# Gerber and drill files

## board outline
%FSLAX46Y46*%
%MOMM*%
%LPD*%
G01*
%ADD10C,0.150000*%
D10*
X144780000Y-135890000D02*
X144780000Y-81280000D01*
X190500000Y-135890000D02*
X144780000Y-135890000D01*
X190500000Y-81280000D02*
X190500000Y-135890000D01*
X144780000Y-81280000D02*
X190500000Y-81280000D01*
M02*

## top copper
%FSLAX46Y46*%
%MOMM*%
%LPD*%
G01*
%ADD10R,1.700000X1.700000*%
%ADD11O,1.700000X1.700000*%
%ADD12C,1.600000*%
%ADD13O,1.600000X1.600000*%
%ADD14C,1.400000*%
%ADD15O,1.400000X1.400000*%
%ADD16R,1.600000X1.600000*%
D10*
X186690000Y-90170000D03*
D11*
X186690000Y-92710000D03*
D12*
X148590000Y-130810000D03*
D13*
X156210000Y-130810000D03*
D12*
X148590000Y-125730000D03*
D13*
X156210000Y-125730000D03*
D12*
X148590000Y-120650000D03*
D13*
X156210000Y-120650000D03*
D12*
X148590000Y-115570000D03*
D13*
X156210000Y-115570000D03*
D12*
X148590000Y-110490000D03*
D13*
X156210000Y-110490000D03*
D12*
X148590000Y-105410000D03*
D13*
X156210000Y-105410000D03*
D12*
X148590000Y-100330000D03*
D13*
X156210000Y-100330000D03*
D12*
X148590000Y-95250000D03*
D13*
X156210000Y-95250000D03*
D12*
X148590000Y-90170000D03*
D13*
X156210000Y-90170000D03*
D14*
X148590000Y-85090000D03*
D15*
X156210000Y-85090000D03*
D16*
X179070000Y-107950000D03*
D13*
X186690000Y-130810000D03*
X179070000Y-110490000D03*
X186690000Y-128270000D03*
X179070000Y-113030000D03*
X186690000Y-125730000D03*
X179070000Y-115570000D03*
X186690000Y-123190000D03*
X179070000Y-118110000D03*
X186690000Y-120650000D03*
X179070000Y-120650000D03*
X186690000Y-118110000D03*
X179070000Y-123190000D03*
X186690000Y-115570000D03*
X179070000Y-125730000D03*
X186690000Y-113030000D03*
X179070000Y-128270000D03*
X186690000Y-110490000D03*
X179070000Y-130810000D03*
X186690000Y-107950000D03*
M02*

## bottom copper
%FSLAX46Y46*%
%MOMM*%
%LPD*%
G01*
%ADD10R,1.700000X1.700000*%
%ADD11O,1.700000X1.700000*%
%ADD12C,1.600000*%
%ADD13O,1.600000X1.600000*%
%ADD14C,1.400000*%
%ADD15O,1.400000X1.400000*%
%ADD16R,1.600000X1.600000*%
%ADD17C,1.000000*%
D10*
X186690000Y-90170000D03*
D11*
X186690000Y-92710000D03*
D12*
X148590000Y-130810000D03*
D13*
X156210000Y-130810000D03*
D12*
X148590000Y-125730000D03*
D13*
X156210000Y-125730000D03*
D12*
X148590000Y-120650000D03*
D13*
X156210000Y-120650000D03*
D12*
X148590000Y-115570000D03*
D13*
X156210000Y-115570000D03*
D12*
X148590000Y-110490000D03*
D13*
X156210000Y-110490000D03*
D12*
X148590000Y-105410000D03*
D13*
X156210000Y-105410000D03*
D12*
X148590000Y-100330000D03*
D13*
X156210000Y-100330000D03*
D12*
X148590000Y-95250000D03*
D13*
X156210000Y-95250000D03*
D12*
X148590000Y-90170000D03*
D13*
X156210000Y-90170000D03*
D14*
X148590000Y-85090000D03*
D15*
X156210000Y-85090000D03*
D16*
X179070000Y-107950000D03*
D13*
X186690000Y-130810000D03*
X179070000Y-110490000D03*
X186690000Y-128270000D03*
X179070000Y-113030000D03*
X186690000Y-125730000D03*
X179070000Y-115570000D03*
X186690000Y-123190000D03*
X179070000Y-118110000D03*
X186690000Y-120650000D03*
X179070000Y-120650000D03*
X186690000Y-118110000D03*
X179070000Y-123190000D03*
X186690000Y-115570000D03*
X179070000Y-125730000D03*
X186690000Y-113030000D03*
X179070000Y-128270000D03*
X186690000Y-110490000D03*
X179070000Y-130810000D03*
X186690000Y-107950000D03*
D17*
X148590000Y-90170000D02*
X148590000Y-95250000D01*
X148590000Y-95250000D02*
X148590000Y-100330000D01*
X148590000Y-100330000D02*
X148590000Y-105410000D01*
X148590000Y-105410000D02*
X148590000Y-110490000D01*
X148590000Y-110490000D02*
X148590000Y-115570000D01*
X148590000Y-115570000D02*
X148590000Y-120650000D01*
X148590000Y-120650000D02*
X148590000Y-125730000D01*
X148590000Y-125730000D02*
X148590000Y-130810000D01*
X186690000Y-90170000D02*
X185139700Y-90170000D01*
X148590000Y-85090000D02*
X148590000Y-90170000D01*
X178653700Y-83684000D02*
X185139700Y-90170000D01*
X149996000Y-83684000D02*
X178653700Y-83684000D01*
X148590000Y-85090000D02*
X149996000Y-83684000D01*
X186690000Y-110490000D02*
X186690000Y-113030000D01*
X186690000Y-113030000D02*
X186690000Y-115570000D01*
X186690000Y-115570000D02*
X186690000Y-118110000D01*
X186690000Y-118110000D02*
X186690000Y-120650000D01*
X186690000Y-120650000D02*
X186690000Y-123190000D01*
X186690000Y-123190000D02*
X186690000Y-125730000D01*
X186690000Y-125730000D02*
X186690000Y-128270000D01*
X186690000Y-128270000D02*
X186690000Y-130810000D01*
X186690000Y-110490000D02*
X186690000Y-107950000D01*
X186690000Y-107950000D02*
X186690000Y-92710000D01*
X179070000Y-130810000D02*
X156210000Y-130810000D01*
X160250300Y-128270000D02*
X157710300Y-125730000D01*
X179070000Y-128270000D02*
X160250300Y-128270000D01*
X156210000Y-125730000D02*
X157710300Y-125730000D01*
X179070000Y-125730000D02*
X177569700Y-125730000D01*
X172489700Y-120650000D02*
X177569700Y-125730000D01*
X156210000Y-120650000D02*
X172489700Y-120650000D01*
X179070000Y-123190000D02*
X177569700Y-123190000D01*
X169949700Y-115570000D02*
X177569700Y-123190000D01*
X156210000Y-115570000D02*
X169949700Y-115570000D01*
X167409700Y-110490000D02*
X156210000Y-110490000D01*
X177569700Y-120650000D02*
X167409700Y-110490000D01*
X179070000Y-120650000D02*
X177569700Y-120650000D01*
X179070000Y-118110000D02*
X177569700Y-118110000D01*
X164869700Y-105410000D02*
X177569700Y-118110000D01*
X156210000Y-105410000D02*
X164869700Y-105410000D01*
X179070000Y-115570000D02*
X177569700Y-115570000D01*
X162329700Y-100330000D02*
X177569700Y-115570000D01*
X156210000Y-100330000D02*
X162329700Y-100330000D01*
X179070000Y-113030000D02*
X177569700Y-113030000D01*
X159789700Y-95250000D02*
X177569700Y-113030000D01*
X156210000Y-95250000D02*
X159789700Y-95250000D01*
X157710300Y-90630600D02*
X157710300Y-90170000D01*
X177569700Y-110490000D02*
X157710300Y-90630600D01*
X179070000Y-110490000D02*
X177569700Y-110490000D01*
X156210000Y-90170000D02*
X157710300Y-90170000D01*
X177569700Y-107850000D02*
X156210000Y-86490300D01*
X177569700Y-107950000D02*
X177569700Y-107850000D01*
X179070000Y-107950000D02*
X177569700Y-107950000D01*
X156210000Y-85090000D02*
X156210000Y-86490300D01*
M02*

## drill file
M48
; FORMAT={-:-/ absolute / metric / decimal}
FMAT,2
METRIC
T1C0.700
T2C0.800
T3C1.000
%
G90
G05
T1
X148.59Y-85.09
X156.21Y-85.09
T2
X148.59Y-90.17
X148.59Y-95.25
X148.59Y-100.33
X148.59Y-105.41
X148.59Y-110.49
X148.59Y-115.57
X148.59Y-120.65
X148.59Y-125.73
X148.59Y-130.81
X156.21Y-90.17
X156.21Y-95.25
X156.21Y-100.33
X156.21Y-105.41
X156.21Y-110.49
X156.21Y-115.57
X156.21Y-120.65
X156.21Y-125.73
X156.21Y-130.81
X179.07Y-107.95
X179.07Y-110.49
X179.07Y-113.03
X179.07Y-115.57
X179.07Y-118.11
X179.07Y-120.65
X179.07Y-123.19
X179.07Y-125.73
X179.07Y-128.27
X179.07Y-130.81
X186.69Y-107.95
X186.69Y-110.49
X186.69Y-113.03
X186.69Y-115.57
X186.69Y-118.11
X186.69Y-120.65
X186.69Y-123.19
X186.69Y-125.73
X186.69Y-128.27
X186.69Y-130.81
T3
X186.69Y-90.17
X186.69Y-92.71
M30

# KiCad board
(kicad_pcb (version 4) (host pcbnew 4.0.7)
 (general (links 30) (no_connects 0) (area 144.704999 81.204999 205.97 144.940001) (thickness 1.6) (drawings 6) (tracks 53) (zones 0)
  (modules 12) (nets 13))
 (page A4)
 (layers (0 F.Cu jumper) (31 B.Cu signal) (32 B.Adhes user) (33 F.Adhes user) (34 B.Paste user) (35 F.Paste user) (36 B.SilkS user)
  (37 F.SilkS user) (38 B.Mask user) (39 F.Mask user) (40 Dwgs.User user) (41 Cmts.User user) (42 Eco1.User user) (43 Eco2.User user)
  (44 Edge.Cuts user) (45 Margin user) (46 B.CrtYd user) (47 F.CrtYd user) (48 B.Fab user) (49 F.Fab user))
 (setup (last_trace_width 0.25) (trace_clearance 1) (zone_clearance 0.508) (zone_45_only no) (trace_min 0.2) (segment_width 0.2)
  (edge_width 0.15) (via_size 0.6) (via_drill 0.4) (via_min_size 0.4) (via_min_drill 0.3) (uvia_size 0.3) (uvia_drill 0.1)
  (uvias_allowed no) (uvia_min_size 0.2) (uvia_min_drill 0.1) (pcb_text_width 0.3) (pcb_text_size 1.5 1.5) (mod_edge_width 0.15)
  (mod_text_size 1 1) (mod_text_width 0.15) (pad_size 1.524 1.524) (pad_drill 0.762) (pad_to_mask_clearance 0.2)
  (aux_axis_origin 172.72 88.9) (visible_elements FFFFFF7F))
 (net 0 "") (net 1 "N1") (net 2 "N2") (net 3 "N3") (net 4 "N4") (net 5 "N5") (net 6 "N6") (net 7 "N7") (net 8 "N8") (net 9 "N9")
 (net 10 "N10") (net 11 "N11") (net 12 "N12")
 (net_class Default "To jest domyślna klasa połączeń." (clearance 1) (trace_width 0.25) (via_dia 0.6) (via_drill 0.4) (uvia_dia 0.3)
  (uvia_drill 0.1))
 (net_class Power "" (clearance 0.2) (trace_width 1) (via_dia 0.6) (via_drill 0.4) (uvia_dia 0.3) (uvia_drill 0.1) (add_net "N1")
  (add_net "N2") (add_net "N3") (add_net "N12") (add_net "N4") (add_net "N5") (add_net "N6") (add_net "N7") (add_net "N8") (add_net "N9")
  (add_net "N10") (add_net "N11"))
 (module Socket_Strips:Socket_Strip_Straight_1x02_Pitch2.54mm (layer F.Cu) (at 186.69 90.17)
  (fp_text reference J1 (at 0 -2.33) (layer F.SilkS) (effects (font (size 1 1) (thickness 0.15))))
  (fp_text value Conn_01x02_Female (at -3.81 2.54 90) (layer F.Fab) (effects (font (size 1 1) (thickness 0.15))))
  (pad 1 thru_hole rect (at 0 0) (size 1.7 1.7) (drill 1) (layers *.Cu *.Mask) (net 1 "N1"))
  (pad 2 thru_hole oval (at 0 2.54) (size 1.7 1.7) (drill 1) (layers *.Cu *.Mask) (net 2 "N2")))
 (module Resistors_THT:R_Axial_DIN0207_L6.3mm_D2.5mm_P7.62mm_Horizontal (layer F.Cu) (at 148.59 130.81)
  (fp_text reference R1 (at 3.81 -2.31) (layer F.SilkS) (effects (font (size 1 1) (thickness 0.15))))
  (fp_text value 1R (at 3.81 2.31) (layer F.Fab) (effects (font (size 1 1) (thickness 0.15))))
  (pad 1 thru_hole circle (at 0 0) (size 1.6 1.6) (drill 0.8) (layers *.Cu *.Mask) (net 1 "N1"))
  (pad 2 thru_hole oval (at 7.62 0) (size 1.6 1.6) (drill 0.8) (layers *.Cu *.Mask) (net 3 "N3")))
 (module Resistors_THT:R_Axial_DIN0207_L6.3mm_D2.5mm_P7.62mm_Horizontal (layer F.Cu) (at 148.59 125.73)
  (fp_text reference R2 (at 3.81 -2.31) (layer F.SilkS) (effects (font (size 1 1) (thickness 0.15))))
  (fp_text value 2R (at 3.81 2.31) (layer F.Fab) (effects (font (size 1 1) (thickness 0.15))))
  (pad 1 thru_hole circle (at 0 0) (size 1.6 1.6) (drill 0.8) (layers *.Cu *.Mask) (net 1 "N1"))
  (pad 2 thru_hole oval (at 7.62 0) (size 1.6 1.6) (drill 0.8) (layers *.Cu *.Mask) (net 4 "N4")))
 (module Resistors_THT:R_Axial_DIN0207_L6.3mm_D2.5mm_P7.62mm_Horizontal (layer F.Cu) (at 148.59 120.65)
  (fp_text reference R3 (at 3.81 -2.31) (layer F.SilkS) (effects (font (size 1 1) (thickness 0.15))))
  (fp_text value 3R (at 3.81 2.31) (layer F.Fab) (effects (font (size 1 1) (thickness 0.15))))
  (pad 1 thru_hole circle (at 0 0) (size 1.6 1.6) (drill 0.8) (layers *.Cu *.Mask) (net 1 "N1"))
  (pad 2 thru_hole oval (at 7.62 0) (size 1.6 1.6) (drill 0.8) (layers *.Cu *.Mask) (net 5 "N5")))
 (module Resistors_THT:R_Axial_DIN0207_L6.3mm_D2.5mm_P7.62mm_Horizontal (layer F.Cu) (at 148.59 115.57)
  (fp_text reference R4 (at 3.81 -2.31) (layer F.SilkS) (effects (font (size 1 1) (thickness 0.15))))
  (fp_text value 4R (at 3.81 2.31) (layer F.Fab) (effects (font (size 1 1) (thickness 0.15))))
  (pad 1 thru_hole circle (at 0 0) (size 1.6 1.6) (drill 0.8) (layers *.Cu *.Mask) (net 1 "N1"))
  (pad 2 thru_hole oval (at 7.62 0) (size 1.6 1.6) (drill 0.8) (layers *.Cu *.Mask) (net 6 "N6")))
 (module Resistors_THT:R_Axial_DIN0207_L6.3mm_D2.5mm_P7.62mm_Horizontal (layer F.Cu) (at 148.59 110.49)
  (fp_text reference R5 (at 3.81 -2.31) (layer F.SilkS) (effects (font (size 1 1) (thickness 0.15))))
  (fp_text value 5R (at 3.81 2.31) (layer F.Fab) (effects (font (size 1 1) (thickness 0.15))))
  (pad 1 thru_hole circle (at 0 0) (size 1.6 1.6) (drill 0.8) (layers *.Cu *.Mask) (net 1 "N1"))
  (pad 2 thru_hole oval (at 7.62 0) (size 1.6 1.6) (drill 0.8) (layers *.Cu *.Mask) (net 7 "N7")))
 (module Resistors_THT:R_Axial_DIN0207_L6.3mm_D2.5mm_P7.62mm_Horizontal (layer F.Cu) (at 148.59 105.41)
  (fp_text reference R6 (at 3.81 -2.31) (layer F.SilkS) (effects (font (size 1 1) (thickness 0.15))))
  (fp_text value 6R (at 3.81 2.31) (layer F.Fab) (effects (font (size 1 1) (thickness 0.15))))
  (pad 1 thru_hole circle (at 0 0) (size 1.6 1.6) (drill 0.8) (layers *.Cu *.Mask) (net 1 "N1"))
  (pad 2 thru_hole oval (at 7.62 0) (size 1.6 1.6) (drill 0.8) (layers *.Cu *.Mask) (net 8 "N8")))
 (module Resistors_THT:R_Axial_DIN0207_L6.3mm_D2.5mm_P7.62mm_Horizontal (layer F.Cu) (at 148.59 100.33)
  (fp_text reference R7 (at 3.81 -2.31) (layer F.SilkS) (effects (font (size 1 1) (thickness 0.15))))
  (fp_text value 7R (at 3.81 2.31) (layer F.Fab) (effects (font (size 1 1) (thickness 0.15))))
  (pad 1 thru_hole circle (at 0 0) (size 1.6 1.6) (drill 0.8) (layers *.Cu *.Mask) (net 1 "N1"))
  (pad 2 thru_hole oval (at 7.62 0) (size 1.6 1.6) (drill 0.8) (layers *.Cu *.Mask) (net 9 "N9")))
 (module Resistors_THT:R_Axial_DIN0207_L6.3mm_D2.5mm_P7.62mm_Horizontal (layer F.Cu) (at 148.59 95.25)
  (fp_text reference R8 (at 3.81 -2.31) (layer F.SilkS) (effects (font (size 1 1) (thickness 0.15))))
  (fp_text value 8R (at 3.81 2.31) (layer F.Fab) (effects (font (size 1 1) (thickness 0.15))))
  (pad 1 thru_hole circle (at 0 0) (size 1.6 1.6) (drill 0.8) (layers *.Cu *.Mask) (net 1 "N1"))
  (pad 2 thru_hole oval (at 7.62 0) (size 1.6 1.6) (drill 0.8) (layers *.Cu *.Mask) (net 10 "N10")))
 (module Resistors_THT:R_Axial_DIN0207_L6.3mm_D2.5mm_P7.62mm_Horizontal (layer F.Cu) (at 148.59 90.17)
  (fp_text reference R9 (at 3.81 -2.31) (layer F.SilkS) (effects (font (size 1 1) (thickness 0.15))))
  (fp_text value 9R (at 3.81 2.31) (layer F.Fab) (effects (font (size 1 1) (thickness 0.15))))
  (pad 1 thru_hole circle (at 0 0) (size 1.6 1.6) (drill 0.8) (layers *.Cu *.Mask) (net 1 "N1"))
  (pad 2 thru_hole oval (at 7.62 0) (size 1.6 1.6) (drill 0.8) (layers *.Cu *.Mask) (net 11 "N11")))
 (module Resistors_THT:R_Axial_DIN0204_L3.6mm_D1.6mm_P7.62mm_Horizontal (layer F.Cu) (at 148.59 85.09)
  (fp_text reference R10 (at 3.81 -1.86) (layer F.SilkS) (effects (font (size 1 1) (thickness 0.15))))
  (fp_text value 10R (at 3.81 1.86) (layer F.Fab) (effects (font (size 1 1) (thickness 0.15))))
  (pad 1 thru_hole circle (at 0 0) (size 1.4 1.4) (drill 0.7) (layers *.Cu *.Mask) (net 1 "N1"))
  (pad 2 thru_hole oval (at 7.62 0) (size 1.4 1.4) (drill 0.7) (layers *.Cu *.Mask) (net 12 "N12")))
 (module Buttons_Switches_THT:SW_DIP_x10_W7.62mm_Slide (layer F.Cu) (at 179.07 107.95)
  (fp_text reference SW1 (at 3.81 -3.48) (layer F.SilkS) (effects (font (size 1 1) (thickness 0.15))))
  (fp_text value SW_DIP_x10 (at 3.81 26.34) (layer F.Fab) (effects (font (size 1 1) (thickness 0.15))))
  (pad 1 thru_hole rect (at 0 0) (size 1.6 1.6) (drill 0.8) (layers *.Cu *.Mask) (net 12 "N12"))
  (pad 11 thru_hole oval (at 7.62 22.86) (size 1.6 1.6) (drill 0.8) (layers *.Cu *.Mask) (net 2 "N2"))
  (pad 2 thru_hole oval (at 0 2.54) (size 1.6 1.6) (drill 0.8) (layers *.Cu *.Mask) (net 11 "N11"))
  (pad 12 thru_hole oval (at 7.62 20.32) (size 1.6 1.6) (drill 0.8) (layers *.Cu *.Mask) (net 2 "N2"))
  (pad 3 thru_hole oval (at 0 5.08) (size 1.6 1.6) (drill 0.8) (layers *.Cu *.Mask) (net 10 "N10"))
  (pad 13 thru_hole oval (at 7.62 17.78) (size 1.6 1.6) (drill 0.8) (layers *.Cu *.Mask) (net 2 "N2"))
  (pad 4 thru_hole oval (at 0 7.62) (size 1.6 1.6) (drill 0.8) (layers *.Cu *.Mask) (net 9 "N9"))
  (pad 14 thru_hole oval (at 7.62 15.24) (size 1.6 1.6) (drill 0.8) (layers *.Cu *.Mask) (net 2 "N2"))
  (pad 5 thru_hole oval (at 0 10.16) (size 1.6 1.6) (drill 0.8) (layers *.Cu *.Mask) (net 8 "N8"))
  (pad 15 thru_hole oval (at 7.62 12.7) (size 1.6 1.6) (drill 0.8) (layers *.Cu *.Mask) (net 2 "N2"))
  (pad 6 thru_hole oval (at 0 12.7) (size 1.6 1.6) (drill 0.8) (layers *.Cu *.Mask) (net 7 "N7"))
  (pad 16 thru_hole oval (at 7.62 10.16) (size 1.6 1.6) (drill 0.8) (layers *.Cu *.Mask) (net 2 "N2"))
  (pad 7 thru_hole oval (at 0 15.24) (size 1.6 1.6) (drill 0.8) (layers *.Cu *.Mask) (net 6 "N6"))
  (pad 17 thru_hole oval (at 7.62 7.62) (size 1.6 1.6) (drill 0.8) (layers *.Cu *.Mask) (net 2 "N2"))
  (pad 8 thru_hole oval (at 0 17.78) (size 1.6 1.6) (drill 0.8) (layers *.Cu *.Mask) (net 5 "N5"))
  (pad 18 thru_hole oval (at 7.62 5.08) (size 1.6 1.6) (drill 0.8) (layers *.Cu *.Mask) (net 2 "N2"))
  (pad 9 thru_hole oval (at 0 20.32) (size 1.6 1.6) (drill 0.8) (layers *.Cu *.Mask) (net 4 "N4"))
  (pad 19 thru_hole oval (at 7.62 2.54) (size 1.6 1.6) (drill 0.8) (layers *.Cu *.Mask) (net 2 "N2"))
  (pad 10 thru_hole oval (at 0 22.86) (size 1.6 1.6) (drill 0.8) (layers *.Cu *.Mask) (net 3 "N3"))
  (pad 20 thru_hole oval (at 7.62 0) (size 1.6 1.6) (drill 0.8) (layers *.Cu *.Mask) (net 2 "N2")))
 (gr_line (start 144.78 135.89) (end 144.78 81.28) (angle 90) (layer Edge.Cuts) (width 0.15))
 (gr_line (start 190.5 135.89) (end 144.78 135.89) (angle 90) (layer Edge.Cuts) (width 0.15))
 (gr_line (start 190.5 81.28) (end 190.5 135.89) (angle 90) (layer Edge.Cuts) (width 0.15))
 (gr_line (start 144.78 81.28) (end 190.5 81.28) (angle 90) (layer Edge.Cuts) (width 0.15))
 (segment (start 148.59 90.17) (end 148.59 95.25) (width 1) (layer B.Cu) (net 1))
 (segment (start 148.59 95.25) (end 148.59 100.33) (width 1) (layer B.Cu) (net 1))
 (segment (start 148.59 100.33) (end 148.59 105.41) (width 1) (layer B.Cu) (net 1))
 (segment (start 148.59 105.41) (end 148.59 110.49) (width 1) (layer B.Cu) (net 1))
 (segment (start 148.59 110.49) (end 148.59 115.57) (width 1) (layer B.Cu) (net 1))
 (segment (start 148.59 115.57) (end 148.59 120.65) (width 1) (layer B.Cu) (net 1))
 (segment (start 148.59 120.65) (end 148.59 125.73) (width 1) (layer B.Cu) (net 1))
 (segment (start 148.59 125.73) (end 148.59 130.81) (width 1) (layer B.Cu) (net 1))
 (segment (start 186.69 90.17) (end 185.1397 90.17) (width 1) (layer B.Cu) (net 1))
 (segment (start 148.59 85.09) (end 148.59 90.17) (width 1) (layer B.Cu) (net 1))
 (segment (start 178.6537 83.684) (end 185.1397 90.17) (width 1) (layer B.Cu) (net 1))
 (segment (start 149.996 83.684) (end 178.6537 83.684) (width 1) (layer B.Cu) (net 1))
 (segment (start 148.59 85.09) (end 149.996 83.684) (width 1) (layer B.Cu) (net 1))
 (segment (start 186.69 110.49) (end 186.69 113.03) (width 1) (layer B.Cu) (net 2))
 (segment (start 186.69 113.03) (end 186.69 115.57) (width 1) (layer B.Cu) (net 2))
 (segment (start 186.69 115.57) (end 186.69 118.11) (width 1) (layer B.Cu) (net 2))
 (segment (start 186.69 118.11) (end 186.69 120.65) (width 1) (layer B.Cu) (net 2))
 (segment (start 186.69 120.65) (end 186.69 123.19) (width 1) (layer B.Cu) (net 2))
 (segment (start 186.69 123.19) (end 186.69 125.73) (width 1) (layer B.Cu) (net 2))
 (segment (start 186.69 125.73) (end 186.69 128.27) (width 1) (layer B.Cu) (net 2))
 (segment (start 186.69 128.27) (end 186.69 130.81) (width 1) (layer B.Cu) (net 2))
 (segment (start 186.69 110.49) (end 186.69 107.95) (width 1) (layer B.Cu) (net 2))
 (segment (start 186.69 107.95) (end 186.69 92.71) (width 1) (layer B.Cu) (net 2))
 (segment (start 179.07 130.81) (end 156.21 130.81) (width 1) (layer B.Cu) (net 3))
 (segment (start 160.2503 128.27) (end 157.7103 125.73) (width 1) (layer B.Cu) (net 4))
 (segment (start 179.07 128.27) (end 160.2503 128.27) (width 1) (layer B.Cu) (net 4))
 (segment (start 156.21 125.73) (end 157.7103 125.73) (width 1) (layer B.Cu) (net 4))
 (segment (start 179.07 125.73) (end 177.5697 125.73) (width 1) (layer B.Cu) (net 5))
 (segment (start 172.4897 120.65) (end 177.5697 125.73) (width 1) (layer B.Cu) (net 5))
 (segment (start 156.21 120.65) (end 172.4897 120.65) (width 1) (layer B.Cu) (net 5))
 (segment (start 179.07 123.19) (end 177.5697 123.19) (width 1) (layer B.Cu) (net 6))
 (segment (start 169.9497 115.57) (end 177.5697 123.19) (width 1) (layer B.Cu) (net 6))
 (segment (start 156.21 115.57) (end 169.9497 115.57) (width 1) (layer B.Cu) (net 6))
 (segment (start 167.4097 110.49) (end 156.21 110.49) (width 1) (layer B.Cu) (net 7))
 (segment (start 177.5697 120.65) (end 167.4097 110.49) (width 1) (layer B.Cu) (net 7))
 (segment (start 179.07 120.65) (end 177.5697 120.65) (width 1) (layer B.Cu) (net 7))
 (segment (start 179.07 118.11) (end 177.5697 118.11) (width 1) (layer B.Cu) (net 8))
 (segment (start 164.8697 105.41) (end 177.5697 118.11) (width 1) (layer B.Cu) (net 8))
 (segment (start 156.21 105.41) (end 164.8697 105.41) (width 1) (layer B.Cu) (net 8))
 (segment (start 179.07 115.57) (end 177.5697 115.57) (width 1) (layer B.Cu) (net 9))
 (segment (start 162.3297 100.33) (end 177.5697 115.57) (width 1) (layer B.Cu) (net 9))
 (segment (start 156.21 100.33) (end 162.3297 100.33) (width 1) (layer B.Cu) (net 9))
 (segment (start 179.07 113.03) (end 177.5697 113.03) (width 1) (layer B.Cu) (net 10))
 (segment (start 159.7897 95.25) (end 177.5697 113.03) (width 1) (layer B.Cu) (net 10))
 (segment (start 156.21 95.25) (end 159.7897 95.25) (width 1) (layer B.Cu) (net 10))
 (segment (start 157.7103 90.6306) (end 157.7103 90.17) (width 1) (layer B.Cu) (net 11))
 (segment (start 177.5697 110.49) (end 157.7103 90.6306) (width 1) (layer B.Cu) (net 11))
 (segment (start 179.07 110.49) (end 177.5697 110.49) (width 1) (layer B.Cu) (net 11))
 (segment (start 156.21 90.17) (end 157.7103 90.17) (width 1) (layer B.Cu) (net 11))
 (segment (start 177.5697 107.85) (end 156.21 86.4903) (width 1) (layer B.Cu) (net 12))
 (segment (start 177.5697 107.95) (end 177.5697 107.85) (width 1) (layer B.Cu) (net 12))
 (segment (start 179.07 107.95) (end 177.5697 107.95) (width 1) (layer B.Cu) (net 12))
 (segment (start 156.21 85.09) (end 156.21 86.4903) (width 1) (layer B.Cu) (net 12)))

